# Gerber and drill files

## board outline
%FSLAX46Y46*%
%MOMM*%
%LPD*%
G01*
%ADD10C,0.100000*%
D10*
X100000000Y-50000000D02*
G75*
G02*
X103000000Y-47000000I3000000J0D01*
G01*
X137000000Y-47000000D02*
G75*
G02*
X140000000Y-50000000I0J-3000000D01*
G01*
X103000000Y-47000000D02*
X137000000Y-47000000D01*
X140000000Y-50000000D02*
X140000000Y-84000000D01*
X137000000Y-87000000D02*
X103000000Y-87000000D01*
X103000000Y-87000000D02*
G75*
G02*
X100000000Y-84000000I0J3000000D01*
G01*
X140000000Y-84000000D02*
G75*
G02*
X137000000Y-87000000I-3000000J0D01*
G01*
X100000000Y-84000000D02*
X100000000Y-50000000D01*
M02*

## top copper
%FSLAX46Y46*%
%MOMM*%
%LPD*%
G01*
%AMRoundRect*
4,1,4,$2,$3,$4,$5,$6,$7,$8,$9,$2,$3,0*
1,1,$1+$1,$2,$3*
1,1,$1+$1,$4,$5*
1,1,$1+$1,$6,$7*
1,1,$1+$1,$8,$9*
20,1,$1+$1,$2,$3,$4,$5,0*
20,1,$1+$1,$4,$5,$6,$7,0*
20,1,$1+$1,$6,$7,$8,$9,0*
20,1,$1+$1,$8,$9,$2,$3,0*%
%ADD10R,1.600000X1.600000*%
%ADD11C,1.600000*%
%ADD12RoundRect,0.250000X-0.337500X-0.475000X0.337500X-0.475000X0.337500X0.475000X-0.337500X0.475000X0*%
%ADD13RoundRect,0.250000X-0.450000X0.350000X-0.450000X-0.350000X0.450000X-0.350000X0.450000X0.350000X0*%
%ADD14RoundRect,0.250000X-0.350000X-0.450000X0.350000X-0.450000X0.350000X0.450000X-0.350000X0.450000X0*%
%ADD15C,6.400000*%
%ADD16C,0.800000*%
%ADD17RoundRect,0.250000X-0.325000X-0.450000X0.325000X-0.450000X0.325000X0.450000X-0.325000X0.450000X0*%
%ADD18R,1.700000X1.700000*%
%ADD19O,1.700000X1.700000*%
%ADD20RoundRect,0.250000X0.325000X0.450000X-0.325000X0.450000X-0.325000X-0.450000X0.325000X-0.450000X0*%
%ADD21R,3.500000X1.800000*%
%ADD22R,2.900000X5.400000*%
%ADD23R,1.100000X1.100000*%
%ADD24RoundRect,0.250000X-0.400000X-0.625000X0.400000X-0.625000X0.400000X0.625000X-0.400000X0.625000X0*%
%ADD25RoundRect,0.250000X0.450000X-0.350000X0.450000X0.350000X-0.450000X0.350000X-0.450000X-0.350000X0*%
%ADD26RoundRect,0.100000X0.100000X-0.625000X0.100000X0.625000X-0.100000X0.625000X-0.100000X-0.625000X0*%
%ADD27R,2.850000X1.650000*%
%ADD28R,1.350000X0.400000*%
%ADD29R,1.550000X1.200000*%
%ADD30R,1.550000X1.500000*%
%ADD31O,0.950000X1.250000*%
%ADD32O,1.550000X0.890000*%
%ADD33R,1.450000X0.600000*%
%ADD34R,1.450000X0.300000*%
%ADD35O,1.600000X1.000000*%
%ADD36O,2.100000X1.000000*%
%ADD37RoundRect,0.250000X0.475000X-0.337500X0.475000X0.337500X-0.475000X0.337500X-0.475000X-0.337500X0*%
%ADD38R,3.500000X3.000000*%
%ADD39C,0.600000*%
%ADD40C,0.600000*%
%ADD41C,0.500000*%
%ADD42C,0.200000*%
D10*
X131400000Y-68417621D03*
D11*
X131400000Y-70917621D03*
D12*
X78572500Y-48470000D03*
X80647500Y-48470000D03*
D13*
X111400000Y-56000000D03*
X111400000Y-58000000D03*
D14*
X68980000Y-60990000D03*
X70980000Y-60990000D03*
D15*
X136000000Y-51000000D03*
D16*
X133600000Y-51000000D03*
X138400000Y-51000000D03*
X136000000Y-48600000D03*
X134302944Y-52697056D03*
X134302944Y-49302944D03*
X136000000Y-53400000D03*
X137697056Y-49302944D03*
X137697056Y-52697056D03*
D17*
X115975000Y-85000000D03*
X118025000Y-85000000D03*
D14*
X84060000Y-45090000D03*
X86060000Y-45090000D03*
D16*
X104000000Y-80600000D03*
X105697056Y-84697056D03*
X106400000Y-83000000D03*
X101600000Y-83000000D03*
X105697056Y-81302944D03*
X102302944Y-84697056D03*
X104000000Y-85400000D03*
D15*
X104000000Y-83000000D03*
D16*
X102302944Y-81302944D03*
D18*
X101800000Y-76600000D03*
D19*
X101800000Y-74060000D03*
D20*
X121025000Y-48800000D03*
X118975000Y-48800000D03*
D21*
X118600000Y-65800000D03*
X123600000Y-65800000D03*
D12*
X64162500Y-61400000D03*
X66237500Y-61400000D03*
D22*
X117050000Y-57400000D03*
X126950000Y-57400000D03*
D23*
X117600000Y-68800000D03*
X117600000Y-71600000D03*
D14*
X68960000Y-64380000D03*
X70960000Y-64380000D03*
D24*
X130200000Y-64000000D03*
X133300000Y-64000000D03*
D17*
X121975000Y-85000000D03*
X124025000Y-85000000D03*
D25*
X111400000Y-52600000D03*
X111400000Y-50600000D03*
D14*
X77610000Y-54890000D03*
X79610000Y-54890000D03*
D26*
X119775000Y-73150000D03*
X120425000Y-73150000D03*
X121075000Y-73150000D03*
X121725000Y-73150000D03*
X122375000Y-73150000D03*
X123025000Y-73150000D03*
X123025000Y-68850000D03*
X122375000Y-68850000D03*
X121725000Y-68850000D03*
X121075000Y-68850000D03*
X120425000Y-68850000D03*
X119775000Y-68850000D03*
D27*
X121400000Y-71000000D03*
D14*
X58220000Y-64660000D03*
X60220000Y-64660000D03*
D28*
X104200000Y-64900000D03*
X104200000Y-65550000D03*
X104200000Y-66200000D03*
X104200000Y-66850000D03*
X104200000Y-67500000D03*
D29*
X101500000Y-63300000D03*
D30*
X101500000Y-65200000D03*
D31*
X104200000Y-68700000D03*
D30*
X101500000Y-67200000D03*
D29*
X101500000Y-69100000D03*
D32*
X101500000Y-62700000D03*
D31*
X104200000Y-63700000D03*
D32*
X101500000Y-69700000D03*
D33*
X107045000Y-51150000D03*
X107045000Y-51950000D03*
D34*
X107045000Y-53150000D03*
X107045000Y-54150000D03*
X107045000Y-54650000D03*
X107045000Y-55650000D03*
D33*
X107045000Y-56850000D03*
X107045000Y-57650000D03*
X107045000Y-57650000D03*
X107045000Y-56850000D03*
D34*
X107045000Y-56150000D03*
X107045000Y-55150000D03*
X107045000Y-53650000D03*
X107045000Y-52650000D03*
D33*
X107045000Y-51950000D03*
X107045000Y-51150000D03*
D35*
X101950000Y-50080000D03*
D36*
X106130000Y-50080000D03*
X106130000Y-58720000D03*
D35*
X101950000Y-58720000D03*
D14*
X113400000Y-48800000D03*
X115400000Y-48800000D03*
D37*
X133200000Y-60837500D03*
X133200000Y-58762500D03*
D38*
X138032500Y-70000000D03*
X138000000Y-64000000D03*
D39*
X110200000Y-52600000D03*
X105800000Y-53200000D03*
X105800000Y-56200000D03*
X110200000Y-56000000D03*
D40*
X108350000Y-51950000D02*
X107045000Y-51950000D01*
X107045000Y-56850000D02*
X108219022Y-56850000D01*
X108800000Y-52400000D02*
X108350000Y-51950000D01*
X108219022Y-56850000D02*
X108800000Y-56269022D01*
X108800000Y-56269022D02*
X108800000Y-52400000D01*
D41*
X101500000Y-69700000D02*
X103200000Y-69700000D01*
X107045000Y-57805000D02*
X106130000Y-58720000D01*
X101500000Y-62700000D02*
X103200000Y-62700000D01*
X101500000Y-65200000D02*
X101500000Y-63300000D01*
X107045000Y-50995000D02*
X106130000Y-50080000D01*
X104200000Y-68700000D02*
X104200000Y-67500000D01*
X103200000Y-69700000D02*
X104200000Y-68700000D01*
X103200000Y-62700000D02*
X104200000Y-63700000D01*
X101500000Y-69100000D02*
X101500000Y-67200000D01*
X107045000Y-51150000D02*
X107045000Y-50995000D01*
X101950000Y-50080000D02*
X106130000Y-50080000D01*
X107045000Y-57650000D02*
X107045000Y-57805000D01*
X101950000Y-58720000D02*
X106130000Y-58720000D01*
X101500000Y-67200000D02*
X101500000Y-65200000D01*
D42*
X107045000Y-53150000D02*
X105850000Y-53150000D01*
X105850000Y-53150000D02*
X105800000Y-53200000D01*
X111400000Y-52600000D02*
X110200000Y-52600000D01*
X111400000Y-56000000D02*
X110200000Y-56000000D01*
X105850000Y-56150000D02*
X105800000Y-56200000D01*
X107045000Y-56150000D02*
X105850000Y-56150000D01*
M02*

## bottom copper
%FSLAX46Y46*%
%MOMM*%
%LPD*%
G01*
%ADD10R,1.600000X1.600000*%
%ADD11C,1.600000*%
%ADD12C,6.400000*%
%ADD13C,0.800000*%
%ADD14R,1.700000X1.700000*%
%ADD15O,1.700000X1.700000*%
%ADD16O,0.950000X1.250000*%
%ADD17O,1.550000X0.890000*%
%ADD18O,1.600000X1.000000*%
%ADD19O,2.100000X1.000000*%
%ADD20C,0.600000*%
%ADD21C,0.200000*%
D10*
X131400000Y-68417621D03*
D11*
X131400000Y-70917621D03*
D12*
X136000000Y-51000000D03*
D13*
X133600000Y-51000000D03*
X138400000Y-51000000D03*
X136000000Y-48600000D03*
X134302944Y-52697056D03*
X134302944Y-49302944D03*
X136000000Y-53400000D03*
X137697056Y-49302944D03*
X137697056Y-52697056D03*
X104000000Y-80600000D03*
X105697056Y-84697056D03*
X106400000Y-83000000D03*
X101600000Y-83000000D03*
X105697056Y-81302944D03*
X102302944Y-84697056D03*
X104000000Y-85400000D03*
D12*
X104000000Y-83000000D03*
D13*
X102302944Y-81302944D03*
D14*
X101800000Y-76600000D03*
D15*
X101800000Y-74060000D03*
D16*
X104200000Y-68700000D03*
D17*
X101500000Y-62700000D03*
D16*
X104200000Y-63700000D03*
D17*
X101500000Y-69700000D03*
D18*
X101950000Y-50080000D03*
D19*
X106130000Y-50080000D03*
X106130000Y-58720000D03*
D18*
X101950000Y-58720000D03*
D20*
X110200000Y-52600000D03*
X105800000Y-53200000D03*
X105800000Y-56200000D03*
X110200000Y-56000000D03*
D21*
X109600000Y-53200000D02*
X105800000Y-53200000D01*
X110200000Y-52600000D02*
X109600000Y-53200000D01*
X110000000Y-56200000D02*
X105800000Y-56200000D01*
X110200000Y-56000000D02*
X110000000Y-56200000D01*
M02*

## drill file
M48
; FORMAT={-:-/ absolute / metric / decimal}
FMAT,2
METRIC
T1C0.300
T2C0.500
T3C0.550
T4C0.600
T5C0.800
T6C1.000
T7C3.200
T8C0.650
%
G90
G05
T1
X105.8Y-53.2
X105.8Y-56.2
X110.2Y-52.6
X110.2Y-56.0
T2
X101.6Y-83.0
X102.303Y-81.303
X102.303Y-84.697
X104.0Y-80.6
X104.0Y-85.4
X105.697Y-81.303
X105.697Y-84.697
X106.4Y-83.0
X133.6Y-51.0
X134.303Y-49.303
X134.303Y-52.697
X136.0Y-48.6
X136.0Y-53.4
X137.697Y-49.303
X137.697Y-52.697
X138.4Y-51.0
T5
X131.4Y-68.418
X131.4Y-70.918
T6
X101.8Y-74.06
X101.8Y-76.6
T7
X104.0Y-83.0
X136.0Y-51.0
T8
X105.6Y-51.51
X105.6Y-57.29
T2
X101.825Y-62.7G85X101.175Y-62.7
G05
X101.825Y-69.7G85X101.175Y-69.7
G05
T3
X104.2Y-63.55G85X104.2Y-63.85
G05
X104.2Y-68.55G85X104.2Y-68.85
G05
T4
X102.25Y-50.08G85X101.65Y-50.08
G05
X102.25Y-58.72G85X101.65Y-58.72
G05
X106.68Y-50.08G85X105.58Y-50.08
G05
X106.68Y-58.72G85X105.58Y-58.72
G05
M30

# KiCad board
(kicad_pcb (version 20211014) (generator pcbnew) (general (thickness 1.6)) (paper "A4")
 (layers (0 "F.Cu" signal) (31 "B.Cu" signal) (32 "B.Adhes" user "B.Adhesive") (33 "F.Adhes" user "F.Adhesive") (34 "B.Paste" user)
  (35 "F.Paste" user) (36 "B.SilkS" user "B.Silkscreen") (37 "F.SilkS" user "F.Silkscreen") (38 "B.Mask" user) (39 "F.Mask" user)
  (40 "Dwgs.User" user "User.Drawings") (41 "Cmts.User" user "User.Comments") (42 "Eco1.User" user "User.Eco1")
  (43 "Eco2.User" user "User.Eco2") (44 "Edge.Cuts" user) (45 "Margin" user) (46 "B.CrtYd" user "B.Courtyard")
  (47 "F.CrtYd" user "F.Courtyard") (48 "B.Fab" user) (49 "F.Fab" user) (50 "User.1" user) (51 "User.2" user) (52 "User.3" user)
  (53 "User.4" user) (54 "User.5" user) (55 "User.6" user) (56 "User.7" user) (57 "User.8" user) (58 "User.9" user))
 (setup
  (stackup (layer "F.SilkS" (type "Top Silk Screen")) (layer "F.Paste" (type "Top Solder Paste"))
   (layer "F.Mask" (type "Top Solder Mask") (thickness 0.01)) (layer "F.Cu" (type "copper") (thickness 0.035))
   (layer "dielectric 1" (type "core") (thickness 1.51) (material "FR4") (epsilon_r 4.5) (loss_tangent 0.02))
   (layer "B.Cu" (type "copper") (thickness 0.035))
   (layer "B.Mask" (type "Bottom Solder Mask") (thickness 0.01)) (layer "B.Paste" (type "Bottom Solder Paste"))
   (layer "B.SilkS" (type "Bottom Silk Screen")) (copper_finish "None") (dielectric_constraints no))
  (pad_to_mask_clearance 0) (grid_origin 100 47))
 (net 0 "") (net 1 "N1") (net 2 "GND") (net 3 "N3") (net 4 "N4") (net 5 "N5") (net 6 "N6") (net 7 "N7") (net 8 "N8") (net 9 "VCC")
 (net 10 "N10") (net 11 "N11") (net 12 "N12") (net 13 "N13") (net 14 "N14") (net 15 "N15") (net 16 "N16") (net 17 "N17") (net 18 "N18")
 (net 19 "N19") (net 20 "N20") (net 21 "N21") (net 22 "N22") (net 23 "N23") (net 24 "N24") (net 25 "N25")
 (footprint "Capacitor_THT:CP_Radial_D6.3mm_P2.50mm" (layer "F.Cu") (at 131.4 68.417621 -90)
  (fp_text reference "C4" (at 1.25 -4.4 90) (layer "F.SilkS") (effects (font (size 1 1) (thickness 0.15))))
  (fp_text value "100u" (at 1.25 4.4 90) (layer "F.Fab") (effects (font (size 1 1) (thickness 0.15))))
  (pad "1" thru_hole rect (at 0 0 270) (size 1.6 1.6) (drill 0.8) (layers *.Cu *.Mask) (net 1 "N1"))
  (pad "2" thru_hole circle (at 2.5 0 270) (size 1.6 1.6) (drill 0.8) (layers *.Cu *.Mask) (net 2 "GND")))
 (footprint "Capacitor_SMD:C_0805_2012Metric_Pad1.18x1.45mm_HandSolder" (layer "F.Cu") (at 79.61 48.47)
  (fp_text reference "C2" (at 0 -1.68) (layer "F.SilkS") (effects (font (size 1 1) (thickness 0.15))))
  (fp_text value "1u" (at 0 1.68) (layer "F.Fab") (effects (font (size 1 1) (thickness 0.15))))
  (pad "1" smd roundrect (at -1.0375 0) (size 1.175 1.45) (layers "F.Cu" "F.Paste" "F.Mask") (roundrect_rratio 0.212766) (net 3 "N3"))
  (pad "2" smd roundrect (at 1.0375 0) (size 1.175 1.45) (layers "F.Cu" "F.Paste" "F.Mask") (roundrect_rratio 0.212766) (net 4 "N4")))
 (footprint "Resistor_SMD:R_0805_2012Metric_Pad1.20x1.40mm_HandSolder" (layer "F.Cu") (at 111.4 57 -90)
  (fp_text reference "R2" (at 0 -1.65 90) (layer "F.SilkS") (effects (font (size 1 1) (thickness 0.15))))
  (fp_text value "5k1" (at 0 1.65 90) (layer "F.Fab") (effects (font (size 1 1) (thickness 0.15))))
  (pad "1" smd roundrect (at -1 0 270) (size 1.2 1.4) (layers "F.Cu" "F.Paste" "F.Mask") (roundrect_rratio 0.208333) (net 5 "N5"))
  (pad "2" smd roundrect (at 1 0 270) (size 1.2 1.4) (layers "F.Cu" "F.Paste" "F.Mask") (roundrect_rratio 0.208333) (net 2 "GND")))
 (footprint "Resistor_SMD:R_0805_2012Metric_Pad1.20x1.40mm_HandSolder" (layer "F.Cu") (at 69.98 60.99)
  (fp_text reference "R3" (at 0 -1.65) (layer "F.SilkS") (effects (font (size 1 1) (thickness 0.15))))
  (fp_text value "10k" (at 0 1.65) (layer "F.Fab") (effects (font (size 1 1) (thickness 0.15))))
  (pad "1" smd roundrect (at -1 0) (size 1.2 1.4) (layers "F.Cu" "F.Paste" "F.Mask") (roundrect_rratio 0.208333) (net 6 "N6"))
  (pad "2" smd roundrect (at 1 0) (size 1.2 1.4) (layers "F.Cu" "F.Paste" "F.Mask") (roundrect_rratio 0.208333) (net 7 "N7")))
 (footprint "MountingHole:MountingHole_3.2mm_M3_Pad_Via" (layer "F.Cu") (at 136 51)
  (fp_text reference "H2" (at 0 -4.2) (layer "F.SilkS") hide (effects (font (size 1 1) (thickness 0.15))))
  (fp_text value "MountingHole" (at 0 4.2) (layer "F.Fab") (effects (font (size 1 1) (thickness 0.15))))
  (pad "1" thru_hole circle (at 0 0) (size 6.4 6.4) (drill 3.2) (layers *.Cu *.Mask))
  (pad "1" thru_hole circle (at -2.4 0) (size 0.8 0.8) (drill 0.5) (layers *.Cu *.Mask))
  (pad "1" thru_hole circle (at 2.4 0) (size 0.8 0.8) (drill 0.5) (layers *.Cu *.Mask))
  (pad "1" thru_hole circle (at 0 -2.4) (size 0.8 0.8) (drill 0.5) (layers *.Cu *.Mask))
  (pad "1" thru_hole circle (at -1.697056 1.697056) (size 0.8 0.8) (drill 0.5) (layers *.Cu *.Mask))
  (pad "1" thru_hole circle (at -1.697056 -1.697056) (size 0.8 0.8) (drill 0.5) (layers *.Cu *.Mask))
  (pad "1" thru_hole circle (at 0 2.4) (size 0.8 0.8) (drill 0.5) (layers *.Cu *.Mask))
  (pad "1" thru_hole circle (at 1.697056 -1.697056) (size 0.8 0.8) (drill 0.5) (layers *.Cu *.Mask))
  (pad "1" thru_hole circle (at 1.697056 1.697056) (size 0.8 0.8) (drill 0.5) (layers *.Cu *.Mask)))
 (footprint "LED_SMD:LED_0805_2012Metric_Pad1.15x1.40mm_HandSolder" (layer "F.Cu") (at 117 85)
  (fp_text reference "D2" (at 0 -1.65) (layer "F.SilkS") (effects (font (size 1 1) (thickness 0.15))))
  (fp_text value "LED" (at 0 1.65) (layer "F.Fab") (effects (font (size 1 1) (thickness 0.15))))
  (pad "1" smd roundrect (at -1.025 0) (size 1.15 1.4) (layers "F.Cu" "F.Paste" "F.Mask") (roundrect_rratio 0.217391) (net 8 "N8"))
  (pad "2" smd roundrect (at 1.025 0) (size 1.15 1.4) (layers "F.Cu" "F.Paste" "F.Mask") (roundrect_rratio 0.217391) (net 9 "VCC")))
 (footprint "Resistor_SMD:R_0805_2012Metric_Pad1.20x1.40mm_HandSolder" (layer "F.Cu") (at 85.06 45.09)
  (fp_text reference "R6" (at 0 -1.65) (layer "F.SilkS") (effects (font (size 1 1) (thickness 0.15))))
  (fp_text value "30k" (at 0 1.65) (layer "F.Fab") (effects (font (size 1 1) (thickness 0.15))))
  (pad "1" smd roundrect (at -1 0) (size 1.2 1.4) (layers "F.Cu" "F.Paste" "F.Mask") (roundrect_rratio 0.208333) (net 1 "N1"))
  (pad "2" smd roundrect (at 1 0) (size 1.2 1.4) (layers "F.Cu" "F.Paste" "F.Mask") (roundrect_rratio 0.208333) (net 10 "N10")))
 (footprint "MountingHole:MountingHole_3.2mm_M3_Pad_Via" (layer "F.Cu") (at 104 83)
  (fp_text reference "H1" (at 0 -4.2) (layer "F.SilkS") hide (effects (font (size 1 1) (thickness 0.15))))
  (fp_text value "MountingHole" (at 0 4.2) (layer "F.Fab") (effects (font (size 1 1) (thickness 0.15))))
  (pad "1" thru_hole circle (at 0 -2.4) (size 0.8 0.8) (drill 0.5) (layers *.Cu *.Mask))
  (pad "1" thru_hole circle (at 1.697056 1.697056) (size 0.8 0.8) (drill 0.5) (layers *.Cu *.Mask))
  (pad "1" thru_hole circle (at 2.4 0) (size 0.8 0.8) (drill 0.5) (layers *.Cu *.Mask))
  (pad "1" thru_hole circle (at -2.4 0) (size 0.8 0.8) (drill 0.5) (layers *.Cu *.Mask))
  (pad "1" thru_hole circle (at 1.697056 -1.697056) (size 0.8 0.8) (drill 0.5) (layers *.Cu *.Mask))
  (pad "1" thru_hole circle (at -1.697056 1.697056) (size 0.8 0.8) (drill 0.5) (layers *.Cu *.Mask))
  (pad "1" thru_hole circle (at 0 2.4) (size 0.8 0.8) (drill 0.5) (layers *.Cu *.Mask))
  (pad "1" thru_hole circle (at 0 0) (size 6.4 6.4) (drill 3.2) (layers *.Cu *.Mask))
  (pad "1" thru_hole circle (at -1.697056 -1.697056) (size 0.8 0.8) (drill 0.5) (layers *.Cu *.Mask)))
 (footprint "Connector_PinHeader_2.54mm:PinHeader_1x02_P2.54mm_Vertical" (layer "F.Cu") (at 101.8 76.6 180)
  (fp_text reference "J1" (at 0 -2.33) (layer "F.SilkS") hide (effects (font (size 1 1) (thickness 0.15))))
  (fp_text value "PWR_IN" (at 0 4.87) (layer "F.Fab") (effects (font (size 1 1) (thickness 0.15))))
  (pad "1" thru_hole rect (at 0 0 180) (size 1.7 1.7) (drill 1) (layers *.Cu *.Mask) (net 2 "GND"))
  (pad "2" thru_hole oval (at 0 2.54 180) (size 1.7 1.7) (drill 1) (layers *.Cu *.Mask) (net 9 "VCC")))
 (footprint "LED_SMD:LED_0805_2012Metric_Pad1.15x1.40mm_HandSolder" (layer "F.Cu") (at 120 48.8 180)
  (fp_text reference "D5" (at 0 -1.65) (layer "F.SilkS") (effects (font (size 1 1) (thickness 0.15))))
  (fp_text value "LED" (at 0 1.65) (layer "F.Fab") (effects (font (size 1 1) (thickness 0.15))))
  (pad "1" smd roundrect (at -1.025 0 180) (size 1.15 1.4) (layers "F.Cu" "F.Paste" "F.Mask") (roundrect_rratio 0.217391) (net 2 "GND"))
  (pad "2" smd roundrect (at 1.025 0 180) (size 1.15 1.4) (layers "F.Cu" "F.Paste" "F.Mask") (roundrect_rratio 0.217391) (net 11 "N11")))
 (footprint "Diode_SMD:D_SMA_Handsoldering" (layer "F.Cu") (at 121.1 65.8)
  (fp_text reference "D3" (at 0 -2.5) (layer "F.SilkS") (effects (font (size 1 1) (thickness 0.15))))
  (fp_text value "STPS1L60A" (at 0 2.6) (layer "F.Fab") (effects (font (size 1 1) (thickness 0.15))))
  (pad "1" smd rect (at -2.5 0) (size 3.5 1.8) (layers "F.Cu" "F.Paste" "F.Mask") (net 4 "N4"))
  (pad "2" smd rect (at 2.5 0) (size 3.5 1.8) (layers "F.Cu" "F.Paste" "F.Mask") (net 1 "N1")))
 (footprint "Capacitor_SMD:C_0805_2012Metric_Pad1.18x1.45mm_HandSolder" (layer "F.Cu") (at 65.2 61.4)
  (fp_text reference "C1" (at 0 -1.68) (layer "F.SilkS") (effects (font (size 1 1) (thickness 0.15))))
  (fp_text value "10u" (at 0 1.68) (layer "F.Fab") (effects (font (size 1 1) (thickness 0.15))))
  (pad "1" smd roundrect (at -1.0375 0) (size 1.175 1.45) (layers "F.Cu" "F.Paste" "F.Mask") (roundrect_rratio 0.212766) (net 9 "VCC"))
  (pad "2" smd roundrect (at 1.0375 0) (size 1.175 1.45) (layers "F.Cu" "F.Paste" "F.Mask") (roundrect_rratio 0.212766) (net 2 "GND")))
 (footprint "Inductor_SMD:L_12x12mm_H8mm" (layer "F.Cu") (at 122 57.4)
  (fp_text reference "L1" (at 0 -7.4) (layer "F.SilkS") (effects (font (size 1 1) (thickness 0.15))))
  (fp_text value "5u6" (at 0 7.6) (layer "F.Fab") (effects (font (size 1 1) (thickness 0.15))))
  (pad "1" smd rect (at -4.95 0) (size 2.9 5.4) (layers "F.Cu" "F.Paste" "F.Mask") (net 3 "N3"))
  (pad "2" smd rect (at 4.95 0) (size 2.9 5.4) (layers "F.Cu" "F.Paste" "F.Mask") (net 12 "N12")))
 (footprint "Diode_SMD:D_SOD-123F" (layer "F.Cu") (at 117.6 70.2 -90)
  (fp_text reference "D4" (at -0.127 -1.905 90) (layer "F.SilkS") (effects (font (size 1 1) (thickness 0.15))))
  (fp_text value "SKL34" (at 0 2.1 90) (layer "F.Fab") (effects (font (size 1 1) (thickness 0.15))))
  (pad "1" smd rect (at -1.4 0 270) (size 1.1 1.1) (layers "F.Cu" "F.Paste" "F.Mask") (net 3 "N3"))
  (pad "2" smd rect (at 1.4 0 270) (size 1.1 1.1) (layers "F.Cu" "F.Paste" "F.Mask") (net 2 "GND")))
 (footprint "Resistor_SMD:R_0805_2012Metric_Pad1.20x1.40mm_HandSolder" (layer "F.Cu") (at 69.96 64.38)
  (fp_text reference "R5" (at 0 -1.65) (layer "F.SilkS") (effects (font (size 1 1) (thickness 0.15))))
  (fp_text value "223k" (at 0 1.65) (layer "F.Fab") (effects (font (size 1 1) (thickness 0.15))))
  (pad "1" smd roundrect (at -1 0) (size 1.2 1.4) (layers "F.Cu" "F.Paste" "F.Mask") (roundrect_rratio 0.208333) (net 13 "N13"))
  (pad "2" smd roundrect (at 1 0) (size 1.2 1.4) (layers "F.Cu" "F.Paste" "F.Mask") (roundrect_rratio 0.208333) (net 10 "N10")))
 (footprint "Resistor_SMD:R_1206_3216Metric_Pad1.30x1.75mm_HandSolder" (layer "F.Cu") (at 131.75 64)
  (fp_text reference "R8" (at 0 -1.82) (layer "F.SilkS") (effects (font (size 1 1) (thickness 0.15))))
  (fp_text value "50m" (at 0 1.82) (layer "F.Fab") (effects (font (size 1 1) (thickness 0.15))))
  (pad "1" smd roundrect (at -1.55 0) (size 1.3 1.75) (layers "F.Cu" "F.Paste" "F.Mask") (roundrect_rratio 0.192308) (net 12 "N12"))
  (pad "2" smd roundrect (at 1.55 0) (size 1.3 1.75) (layers "F.Cu" "F.Paste" "F.Mask") (roundrect_rratio 0.192308) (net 1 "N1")))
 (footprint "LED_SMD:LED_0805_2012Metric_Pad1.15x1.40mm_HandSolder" (layer "F.Cu") (at 123 85)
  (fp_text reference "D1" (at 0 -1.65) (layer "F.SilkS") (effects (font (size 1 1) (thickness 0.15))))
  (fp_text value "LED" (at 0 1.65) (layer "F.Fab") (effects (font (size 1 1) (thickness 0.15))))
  (pad "1" smd roundrect (at -1.025 0) (size 1.15 1.4) (layers "F.Cu" "F.Paste" "F.Mask") (roundrect_rratio 0.217391) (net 6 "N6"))
  (pad "2" smd roundrect (at 1.025 0) (size 1.15 1.4) (layers "F.Cu" "F.Paste" "F.Mask") (roundrect_rratio 0.217391) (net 9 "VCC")))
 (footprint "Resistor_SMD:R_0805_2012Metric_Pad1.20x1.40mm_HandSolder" (layer "F.Cu") (at 111.4 51.6 90)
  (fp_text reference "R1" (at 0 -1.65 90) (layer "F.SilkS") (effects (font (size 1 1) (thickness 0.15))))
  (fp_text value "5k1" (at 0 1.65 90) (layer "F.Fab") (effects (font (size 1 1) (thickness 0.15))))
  (pad "1" smd roundrect (at -1 0 90) (size 1.2 1.4) (layers "F.Cu" "F.Paste" "F.Mask") (roundrect_rratio 0.208333) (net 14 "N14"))
  (pad "2" smd roundrect (at 1 0 90) (size 1.2 1.4) (layers "F.Cu" "F.Paste" "F.Mask") (roundrect_rratio 0.208333) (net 2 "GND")))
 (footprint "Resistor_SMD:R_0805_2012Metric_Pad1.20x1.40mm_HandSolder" (layer "F.Cu") (at 78.61 54.89)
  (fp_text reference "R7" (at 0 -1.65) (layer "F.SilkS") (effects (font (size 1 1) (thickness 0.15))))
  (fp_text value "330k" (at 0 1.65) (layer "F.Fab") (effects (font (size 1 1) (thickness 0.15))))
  (pad "1" smd roundrect (at -1 0) (size 1.2 1.4) (layers "F.Cu" "F.Paste" "F.Mask") (roundrect_rratio 0.208333) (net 10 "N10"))
  (pad "2" smd roundrect (at 1 0) (size 1.2 1.4) (layers "F.Cu" "F.Paste" "F.Mask") (roundrect_rratio 0.208333) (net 2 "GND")))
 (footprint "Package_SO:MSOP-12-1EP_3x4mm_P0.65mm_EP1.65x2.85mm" (layer "F.Cu") (at 121.4 71 90)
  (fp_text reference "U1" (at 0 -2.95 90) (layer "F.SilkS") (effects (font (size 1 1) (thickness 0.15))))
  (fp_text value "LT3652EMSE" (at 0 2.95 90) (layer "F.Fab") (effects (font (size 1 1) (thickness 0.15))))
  (pad "" smd roundrect (at -0.41 0.71 90) (size 0.67 1.15) (layers "F.Paste") (roundrect_rratio 0.25))
  (pad "" smd roundrect (at -0.41 -0.71 90) (size 0.67 1.15) (layers "F.Paste") (roundrect_rratio 0.25))
  (pad "" smd roundrect (at 0.41 -0.71 90) (size 0.67 1.15) (layers "F.Paste") (roundrect_rratio 0.25))
  (pad "" smd roundrect (at 0.41 0.71 90) (size 0.67 1.15) (layers "F.Paste") (roundrect_rratio 0.25))
  (pad "1" smd roundrect (at -2.15 -1.625 90) (size 1.45 0.4) (layers "F.Cu" "F.Paste" "F.Mask") (roundrect_rratio 0.25) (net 9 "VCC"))
  (pad "2" smd roundrect (at -2.15 -0.975 90) (size 1.45 0.4) (layers "F.Cu" "F.Paste" "F.Mask") (roundrect_rratio 0.25) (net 9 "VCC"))
  (pad "3" smd roundrect (at -2.15 -0.325 90) (size 1.45 0.4) (layers "F.Cu" "F.Paste" "F.Mask") (roundrect_rratio 0.25) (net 9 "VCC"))
  (pad "4" smd roundrect (at -2.15 0.325 90) (size 1.45 0.4) (layers "F.Cu" "F.Paste" "F.Mask") (roundrect_rratio 0.25) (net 7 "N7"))
  (pad "5" smd roundrect (at -2.15 0.975 90) (size 1.45 0.4) (layers "F.Cu" "F.Paste" "F.Mask") (roundrect_rratio 0.25) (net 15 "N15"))
  (pad "6" smd roundrect (at -2.15 1.625 90) (size 1.45 0.4) (layers "F.Cu" "F.Paste" "F.Mask") (roundrect_rratio 0.25) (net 2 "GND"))
  (pad "7" smd roundrect (at 2.15 1.625 90) (size 1.45 0.4) (layers "F.Cu" "F.Paste" "F.Mask") (roundrect_rratio 0.25) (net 13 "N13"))
  (pad "8" smd roundrect (at 2.15 0.975 90) (size 1.45 0.4) (layers "F.Cu" "F.Paste" "F.Mask") (roundrect_rratio 0.25) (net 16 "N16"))
  (pad "9" smd roundrect (at 2.15 0.325 90) (size 1.45 0.4) (layers "F.Cu" "F.Paste" "F.Mask") (roundrect_rratio 0.25) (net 1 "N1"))
  (pad "10" smd roundrect (at 2.15 -0.325 90) (size 1.45 0.4) (layers "F.Cu" "F.Paste" "F.Mask") (roundrect_rratio 0.25) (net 12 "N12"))
  (pad "11" smd roundrect (at 2.15 -0.975 90) (size 1.45 0.4) (layers "F.Cu" "F.Paste" "F.Mask") (roundrect_rratio 0.25) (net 4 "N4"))
  (pad "12" smd roundrect (at 2.15 -1.625 90) (size 1.45 0.4) (layers "F.Cu" "F.Paste" "F.Mask") (roundrect_rratio 0.25) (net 3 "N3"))
  (pad "13" smd rect (at 0 0 90) (size 1.65 2.85) (layers "F.Cu" "F.Mask") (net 2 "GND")))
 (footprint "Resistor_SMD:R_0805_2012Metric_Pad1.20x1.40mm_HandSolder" (layer "F.Cu") (at 59.22 64.66)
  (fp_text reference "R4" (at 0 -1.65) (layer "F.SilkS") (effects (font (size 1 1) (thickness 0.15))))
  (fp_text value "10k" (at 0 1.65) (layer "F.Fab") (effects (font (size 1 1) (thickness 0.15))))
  (pad "1" smd roundrect (at -1 0) (size 1.2 1.4) (layers "F.Cu" "F.Paste" "F.Mask") (roundrect_rratio 0.208333) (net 8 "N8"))
  (pad "2" smd roundrect (at 1 0) (size 1.2 1.4) (layers "F.Cu" "F.Paste" "F.Mask") (roundrect_rratio 0.208333) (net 15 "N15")))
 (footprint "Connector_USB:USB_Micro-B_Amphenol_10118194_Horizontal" (layer "F.Cu") (at 102.8 66.2 -90)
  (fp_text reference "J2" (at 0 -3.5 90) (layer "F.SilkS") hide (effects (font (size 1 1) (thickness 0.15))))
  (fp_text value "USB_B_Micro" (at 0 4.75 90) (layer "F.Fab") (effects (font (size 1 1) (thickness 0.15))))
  (pad "" smd oval (at -2.5 -1.4 270) (size 1.25 0.95) (layers "F.Paste"))
  (pad "" smd oval (at 3.5 1.3 270) (size 0.89 1.55) (layers "F.Paste"))
  (pad "" smd oval (at 2.5 -1.4 270) (size 1.25 0.95) (layers "F.Paste"))
  (pad "" smd oval (at -3.5 1.3 270) (size 0.89 1.55) (layers "F.Paste"))
  (pad "1" smd rect (at -1.3 -1.4 270) (size 0.4 1.35) (layers "F.Cu" "F.Paste" "F.Mask") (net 9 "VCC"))
  (pad "2" smd rect (at -0.65 -1.4 270) (size 0.4 1.35) (layers "F.Cu" "F.Paste" "F.Mask") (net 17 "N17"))
  (pad "3" smd rect (at 0 -1.4 270) (size 0.4 1.35) (layers "F.Cu" "F.Paste" "F.Mask") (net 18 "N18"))
  (pad "4" smd rect (at 0.65 -1.4 270) (size 0.4 1.35) (layers "F.Cu" "F.Paste" "F.Mask") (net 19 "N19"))
  (pad "5" smd rect (at 1.3 -1.4 270) (size 0.4 1.35) (layers "F.Cu" "F.Paste" "F.Mask") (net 2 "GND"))
  (pad "6" smd rect (at -2.9 1.3 270) (size 1.2 1.55) (layers "F.Cu" "F.Paste" "F.Mask") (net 2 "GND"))
  (pad "6" smd rect (at -1 1.3 270) (size 1.5 1.55) (layers "F.Cu" "F.Paste" "F.Mask") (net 2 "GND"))
  (pad "6" thru_hole oval (at 2.5 -1.4 270) (size 1.25 0.95) (drill oval 0.85 0.55) (layers *.Cu *.Mask) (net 2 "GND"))
  (pad "6" smd rect (at 1 1.3 270) (size 1.5 1.55) (layers "F.Cu" "F.Paste" "F.Mask") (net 2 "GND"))
  (pad "6" smd rect (at 2.9 1.3 270) (size 1.2 1.55) (layers "F.Cu" "F.Paste" "F.Mask") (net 2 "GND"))
  (pad "6" thru_hole oval (at -3.5 1.3 270) (size 0.89 1.55) (drill oval 0.5 1.15) (layers *.Cu *.Mask) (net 2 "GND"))
  (pad "6" thru_hole oval (at -2.5 -1.4 270) (size 1.25 0.95) (drill oval 0.85 0.55) (layers *.Cu *.Mask) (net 2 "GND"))
  (pad "6" thru_hole oval (at 3.5 1.3 270) (size 0.89 1.55) (drill oval 0.5 1.15) (layers *.Cu *.Mask) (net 2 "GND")))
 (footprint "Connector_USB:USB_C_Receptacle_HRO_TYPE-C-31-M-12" (layer "F.Cu") (at 103 54.4 -90)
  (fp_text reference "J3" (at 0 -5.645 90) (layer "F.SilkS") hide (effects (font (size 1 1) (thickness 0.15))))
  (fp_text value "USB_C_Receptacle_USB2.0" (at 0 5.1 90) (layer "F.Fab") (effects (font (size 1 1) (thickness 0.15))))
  (pad "" np_thru_hole circle (at 2.89 -2.6 270) (size 0.65 0.65) (drill 0.65) (layers *.Cu *.Mask))
  (pad "" np_thru_hole circle (at -2.89 -2.6 270) (size 0.65 0.65) (drill 0.65) (layers *.Cu *.Mask))
  (pad "A1" smd rect (at -3.25 -4.045 270) (size 0.6 1.45) (layers "F.Cu" "F.Paste" "F.Mask") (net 2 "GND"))
  (pad "A4" smd rect (at -2.45 -4.045 270) (size 0.6 1.45) (layers "F.Cu" "F.Paste" "F.Mask") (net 9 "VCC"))
  (pad "A5" smd rect (at -1.25 -4.045 270) (size 0.3 1.45) (layers "F.Cu" "F.Paste" "F.Mask") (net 14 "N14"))
  (pad "A6" smd rect (at -0.25 -4.045 270) (size 0.3 1.45) (layers "F.Cu" "F.Paste" "F.Mask") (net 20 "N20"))
  (pad "A7" smd rect (at 0.25 -4.045 270) (size 0.3 1.45) (layers "F.Cu" "F.Paste" "F.Mask") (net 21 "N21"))
  (pad "A8" smd rect (at 1.25 -4.045 270) (size 0.3 1.45) (layers "F.Cu" "F.Paste" "F.Mask") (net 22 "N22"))
  (pad "A9" smd rect (at 2.45 -4.045 270) (size 0.6 1.45) (layers "F.Cu" "F.Paste" "F.Mask") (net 9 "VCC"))
  (pad "A12" smd rect (at 3.25 -4.045 270) (size 0.6 1.45) (layers "F.Cu" "F.Paste" "F.Mask") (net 2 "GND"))
  (pad "B1" smd rect (at 3.25 -4.045 270) (size 0.6 1.45) (layers "F.Cu" "F.Paste" "F.Mask") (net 2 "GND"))
  (pad "B4" smd rect (at 2.45 -4.045 270) (size 0.6 1.45) (layers "F.Cu" "F.Paste" "F.Mask") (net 9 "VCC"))
  (pad "B5" smd rect (at 1.75 -4.045 270) (size 0.3 1.45) (layers "F.Cu" "F.Paste" "F.Mask") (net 5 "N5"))
  (pad "B6" smd rect (at 0.75 -4.045 270) (size 0.3 1.45) (layers "F.Cu" "F.Paste" "F.Mask") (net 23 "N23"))
  (pad "B7" smd rect (at -0.75 -4.045 270) (size 0.3 1.45) (layers "F.Cu" "F.Paste" "F.Mask") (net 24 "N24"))
  (pad "B8" smd rect (at -1.75 -4.045 270) (size 0.3 1.45) (layers "F.Cu" "F.Paste" "F.Mask") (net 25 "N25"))
  (pad "B9" smd rect (at -2.45 -4.045 270) (size 0.6 1.45) (layers "F.Cu" "F.Paste" "F.Mask") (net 9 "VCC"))
  (pad "B12" smd rect (at -3.25 -4.045 270) (size 0.6 1.45) (layers "F.Cu" "F.Paste" "F.Mask") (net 2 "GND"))
  (pad "S1" thru_hole oval (at -4.32 1.05 270) (size 1 1.6) (drill oval 0.6 1.2) (layers *.Cu *.Mask) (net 2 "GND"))
  (pad "S1" thru_hole oval (at -4.32 -3.13 270) (size 1 2.1) (drill oval 0.6 1.7) (layers *.Cu *.Mask) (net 2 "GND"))
  (pad "S1" thru_hole oval (at 4.32 -3.13 270) (size 1 2.1) (drill oval 0.6 1.7) (layers *.Cu *.Mask) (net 2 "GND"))
  (pad "S1" thru_hole oval (at 4.32 1.05 270) (size 1 1.6) (drill oval 0.6 1.2) (layers *.Cu *.Mask) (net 2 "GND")))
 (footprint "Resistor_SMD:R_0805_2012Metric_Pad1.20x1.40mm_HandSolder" (layer "F.Cu") (at 114.4 48.8)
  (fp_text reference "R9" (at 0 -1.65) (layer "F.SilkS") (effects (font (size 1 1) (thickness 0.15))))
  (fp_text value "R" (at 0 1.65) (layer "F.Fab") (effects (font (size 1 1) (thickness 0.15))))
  (pad "1" smd roundrect (at -1 0) (size 1.2 1.4) (layers "F.Cu" "F.Paste" "F.Mask") (roundrect_rratio 0.208333) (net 9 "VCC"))
  (pad "2" smd roundrect (at 1 0) (size 1.2 1.4) (layers "F.Cu" "F.Paste" "F.Mask") (roundrect_rratio 0.208333) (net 11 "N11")))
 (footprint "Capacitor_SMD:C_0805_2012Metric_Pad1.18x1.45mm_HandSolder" (layer "F.Cu") (at 133.2 59.8 90)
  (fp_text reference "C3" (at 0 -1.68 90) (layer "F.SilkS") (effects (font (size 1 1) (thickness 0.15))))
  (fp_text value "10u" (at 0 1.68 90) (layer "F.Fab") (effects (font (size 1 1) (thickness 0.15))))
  (pad "1" smd roundrect (at -1.0375 0 90) (size 1.175 1.45) (layers "F.Cu" "F.Paste" "F.Mask") (roundrect_rratio 0.212766) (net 1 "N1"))
  (pad "2" smd roundrect (at 1.0375 0 90) (size 1.175 1.45) (layers "F.Cu" "F.Paste" "F.Mask") (roundrect_rratio 0.212766) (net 2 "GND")))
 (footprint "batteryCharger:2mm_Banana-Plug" (layer "F.Cu") (at 139.7825 70 -90)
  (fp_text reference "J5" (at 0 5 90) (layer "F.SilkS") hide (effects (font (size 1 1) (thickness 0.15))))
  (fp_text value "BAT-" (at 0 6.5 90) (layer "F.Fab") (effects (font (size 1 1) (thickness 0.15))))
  (pad "1" smd rect (at 0 1.75 270) (size 3 3.5) (layers "F.Cu" "F.Paste" "F.Mask") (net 2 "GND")))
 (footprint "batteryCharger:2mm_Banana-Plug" (layer "F.Cu") (at 139.75 64 -90)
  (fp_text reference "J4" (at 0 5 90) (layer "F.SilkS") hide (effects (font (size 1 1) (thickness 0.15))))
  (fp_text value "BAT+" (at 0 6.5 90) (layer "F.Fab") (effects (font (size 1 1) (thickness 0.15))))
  (pad "1" smd rect (at 0 1.75 270) (size 3 3.5) (layers "F.Cu" "F.Paste" "F.Mask") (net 1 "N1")))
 (gr_arc (start 100 50) (mid 100.87868 47.87868) (end 103 47) (layer "Edge.Cuts") (width 0.1))
 (gr_arc (start 137 47) (mid 139.12132 47.87868) (end 140 50) (layer "Edge.Cuts") (width 0.1))
 (gr_line (start 103 47) (end 137 47) (layer "Edge.Cuts") (width 0.1))
 (gr_line (start 140 50) (end 140 84) (layer "Edge.Cuts") (width 0.1))
 (gr_line (start 137 87) (end 103 87) (layer "Edge.Cuts") (width 0.1))
 (gr_arc (start 103 87) (mid 100.87868 86.12132) (end 100 84) (layer "Edge.Cuts") (width 0.1))
 (gr_arc (start 140 84) (mid 139.12132 86.12132) (end 137 87) (layer "Edge.Cuts") (width 0.1))
 (gr_line (start 100 84) (end 100 50) (layer "Edge.Cuts") (width 0.1))
 (segment (start 108.35 51.95) (end 107.045 51.95) (width 0.6) (layer "F.Cu") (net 9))
 (segment (start 107.045 56.85) (end 108.219022 56.85) (width 0.6) (layer "F.Cu") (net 9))
 (segment (start 108.8 52.4) (end 108.35 51.95) (width 0.6) (layer "F.Cu") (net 9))
 (segment (start 108.219022 56.85) (end 108.8 56.269022) (width 0.6) (layer "F.Cu") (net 9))
 (segment (start 108.8 56.269022) (end 108.8 52.4) (width 0.6) (layer "F.Cu") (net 9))
 (segment (start 101.5 69.7) (end 103.2 69.7) (width 0.5) (layer "F.Cu") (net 2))
 (segment (start 107.045 57.805) (end 106.13 58.72) (width 0.5) (layer "F.Cu") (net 2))
 (segment (start 101.5 62.7) (end 103.2 62.7) (width 0.5) (layer "F.Cu") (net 2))
 (segment (start 101.5 65.2) (end 101.5 63.3) (width 0.5) (layer "F.Cu") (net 2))
 (segment (start 107.045 50.995) (end 106.13 50.08) (width 0.5) (layer "F.Cu") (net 2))
 (segment (start 104.2 68.7) (end 104.2 67.5) (width 0.5) (layer "F.Cu") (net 2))
 (segment (start 103.2 69.7) (end 104.2 68.7) (width 0.5) (layer "F.Cu") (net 2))
 (segment (start 103.2 62.7) (end 104.2 63.7) (width 0.5) (layer "F.Cu") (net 2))
 (segment (start 101.5 69.1) (end 101.5 67.2) (width 0.5) (layer "F.Cu") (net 2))
 (segment (start 107.045 51.15) (end 107.045 50.995) (width 0.5) (layer "F.Cu") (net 2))
 (segment (start 101.95 50.08) (end 106.13 50.08) (width 0.5) (layer "F.Cu") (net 2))
 (segment (start 107.045 57.65) (end 107.045 57.805) (width 0.5) (layer "F.Cu") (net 2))
 (segment (start 101.95 58.72) (end 106.13 58.72) (width 0.5) (layer "F.Cu") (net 2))
 (segment (start 101.5 67.2) (end 101.5 65.2) (width 0.5) (layer "F.Cu") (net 2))
 (segment (start 107.045 53.15) (end 105.85 53.15) (width 0.2) (layer "F.Cu") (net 14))
 (segment (start 105.85 53.15) (end 105.8 53.2) (width 0.2) (layer "F.Cu") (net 14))
 (segment (start 111.4 52.6) (end 110.2 52.6) (width 0.2) (layer "F.Cu") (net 14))
 (via (at 110.2 52.6) (size 0.6) (drill 0.3) (layers "F.Cu" "B.Cu") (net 14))
 (via (at 105.8 53.2) (size 0.6) (drill 0.3) (layers "F.Cu" "B.Cu") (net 14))
 (segment (start 109.6 53.2) (end 105.8 53.2) (width 0.2) (layer "B.Cu") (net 14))
 (segment (start 110.2 52.6) (end 109.6 53.2) (width 0.2) (layer "B.Cu") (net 14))
 (segment (start 111.4 56) (end 110.2 56) (width 0.2) (layer "F.Cu") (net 5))
 (segment (start 105.85 56.15) (end 105.8 56.2) (width 0.2) (layer "F.Cu") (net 5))
 (segment (start 107.045 56.15) (end 105.85 56.15) (width 0.2) (layer "F.Cu") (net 5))
 (via (at 105.8 56.2) (size 0.6) (drill 0.3) (layers "F.Cu" "B.Cu") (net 5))
 (via (at 110.2 56) (size 0.6) (drill 0.3) (layers "F.Cu" "B.Cu") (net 5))
 (segment (start 110 56.2) (end 105.8 56.2) (width 0.2) (layer "B.Cu") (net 5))
 (segment (start 110.2 56) (end 110 56.2) (width 0.2) (layer "B.Cu") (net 5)))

